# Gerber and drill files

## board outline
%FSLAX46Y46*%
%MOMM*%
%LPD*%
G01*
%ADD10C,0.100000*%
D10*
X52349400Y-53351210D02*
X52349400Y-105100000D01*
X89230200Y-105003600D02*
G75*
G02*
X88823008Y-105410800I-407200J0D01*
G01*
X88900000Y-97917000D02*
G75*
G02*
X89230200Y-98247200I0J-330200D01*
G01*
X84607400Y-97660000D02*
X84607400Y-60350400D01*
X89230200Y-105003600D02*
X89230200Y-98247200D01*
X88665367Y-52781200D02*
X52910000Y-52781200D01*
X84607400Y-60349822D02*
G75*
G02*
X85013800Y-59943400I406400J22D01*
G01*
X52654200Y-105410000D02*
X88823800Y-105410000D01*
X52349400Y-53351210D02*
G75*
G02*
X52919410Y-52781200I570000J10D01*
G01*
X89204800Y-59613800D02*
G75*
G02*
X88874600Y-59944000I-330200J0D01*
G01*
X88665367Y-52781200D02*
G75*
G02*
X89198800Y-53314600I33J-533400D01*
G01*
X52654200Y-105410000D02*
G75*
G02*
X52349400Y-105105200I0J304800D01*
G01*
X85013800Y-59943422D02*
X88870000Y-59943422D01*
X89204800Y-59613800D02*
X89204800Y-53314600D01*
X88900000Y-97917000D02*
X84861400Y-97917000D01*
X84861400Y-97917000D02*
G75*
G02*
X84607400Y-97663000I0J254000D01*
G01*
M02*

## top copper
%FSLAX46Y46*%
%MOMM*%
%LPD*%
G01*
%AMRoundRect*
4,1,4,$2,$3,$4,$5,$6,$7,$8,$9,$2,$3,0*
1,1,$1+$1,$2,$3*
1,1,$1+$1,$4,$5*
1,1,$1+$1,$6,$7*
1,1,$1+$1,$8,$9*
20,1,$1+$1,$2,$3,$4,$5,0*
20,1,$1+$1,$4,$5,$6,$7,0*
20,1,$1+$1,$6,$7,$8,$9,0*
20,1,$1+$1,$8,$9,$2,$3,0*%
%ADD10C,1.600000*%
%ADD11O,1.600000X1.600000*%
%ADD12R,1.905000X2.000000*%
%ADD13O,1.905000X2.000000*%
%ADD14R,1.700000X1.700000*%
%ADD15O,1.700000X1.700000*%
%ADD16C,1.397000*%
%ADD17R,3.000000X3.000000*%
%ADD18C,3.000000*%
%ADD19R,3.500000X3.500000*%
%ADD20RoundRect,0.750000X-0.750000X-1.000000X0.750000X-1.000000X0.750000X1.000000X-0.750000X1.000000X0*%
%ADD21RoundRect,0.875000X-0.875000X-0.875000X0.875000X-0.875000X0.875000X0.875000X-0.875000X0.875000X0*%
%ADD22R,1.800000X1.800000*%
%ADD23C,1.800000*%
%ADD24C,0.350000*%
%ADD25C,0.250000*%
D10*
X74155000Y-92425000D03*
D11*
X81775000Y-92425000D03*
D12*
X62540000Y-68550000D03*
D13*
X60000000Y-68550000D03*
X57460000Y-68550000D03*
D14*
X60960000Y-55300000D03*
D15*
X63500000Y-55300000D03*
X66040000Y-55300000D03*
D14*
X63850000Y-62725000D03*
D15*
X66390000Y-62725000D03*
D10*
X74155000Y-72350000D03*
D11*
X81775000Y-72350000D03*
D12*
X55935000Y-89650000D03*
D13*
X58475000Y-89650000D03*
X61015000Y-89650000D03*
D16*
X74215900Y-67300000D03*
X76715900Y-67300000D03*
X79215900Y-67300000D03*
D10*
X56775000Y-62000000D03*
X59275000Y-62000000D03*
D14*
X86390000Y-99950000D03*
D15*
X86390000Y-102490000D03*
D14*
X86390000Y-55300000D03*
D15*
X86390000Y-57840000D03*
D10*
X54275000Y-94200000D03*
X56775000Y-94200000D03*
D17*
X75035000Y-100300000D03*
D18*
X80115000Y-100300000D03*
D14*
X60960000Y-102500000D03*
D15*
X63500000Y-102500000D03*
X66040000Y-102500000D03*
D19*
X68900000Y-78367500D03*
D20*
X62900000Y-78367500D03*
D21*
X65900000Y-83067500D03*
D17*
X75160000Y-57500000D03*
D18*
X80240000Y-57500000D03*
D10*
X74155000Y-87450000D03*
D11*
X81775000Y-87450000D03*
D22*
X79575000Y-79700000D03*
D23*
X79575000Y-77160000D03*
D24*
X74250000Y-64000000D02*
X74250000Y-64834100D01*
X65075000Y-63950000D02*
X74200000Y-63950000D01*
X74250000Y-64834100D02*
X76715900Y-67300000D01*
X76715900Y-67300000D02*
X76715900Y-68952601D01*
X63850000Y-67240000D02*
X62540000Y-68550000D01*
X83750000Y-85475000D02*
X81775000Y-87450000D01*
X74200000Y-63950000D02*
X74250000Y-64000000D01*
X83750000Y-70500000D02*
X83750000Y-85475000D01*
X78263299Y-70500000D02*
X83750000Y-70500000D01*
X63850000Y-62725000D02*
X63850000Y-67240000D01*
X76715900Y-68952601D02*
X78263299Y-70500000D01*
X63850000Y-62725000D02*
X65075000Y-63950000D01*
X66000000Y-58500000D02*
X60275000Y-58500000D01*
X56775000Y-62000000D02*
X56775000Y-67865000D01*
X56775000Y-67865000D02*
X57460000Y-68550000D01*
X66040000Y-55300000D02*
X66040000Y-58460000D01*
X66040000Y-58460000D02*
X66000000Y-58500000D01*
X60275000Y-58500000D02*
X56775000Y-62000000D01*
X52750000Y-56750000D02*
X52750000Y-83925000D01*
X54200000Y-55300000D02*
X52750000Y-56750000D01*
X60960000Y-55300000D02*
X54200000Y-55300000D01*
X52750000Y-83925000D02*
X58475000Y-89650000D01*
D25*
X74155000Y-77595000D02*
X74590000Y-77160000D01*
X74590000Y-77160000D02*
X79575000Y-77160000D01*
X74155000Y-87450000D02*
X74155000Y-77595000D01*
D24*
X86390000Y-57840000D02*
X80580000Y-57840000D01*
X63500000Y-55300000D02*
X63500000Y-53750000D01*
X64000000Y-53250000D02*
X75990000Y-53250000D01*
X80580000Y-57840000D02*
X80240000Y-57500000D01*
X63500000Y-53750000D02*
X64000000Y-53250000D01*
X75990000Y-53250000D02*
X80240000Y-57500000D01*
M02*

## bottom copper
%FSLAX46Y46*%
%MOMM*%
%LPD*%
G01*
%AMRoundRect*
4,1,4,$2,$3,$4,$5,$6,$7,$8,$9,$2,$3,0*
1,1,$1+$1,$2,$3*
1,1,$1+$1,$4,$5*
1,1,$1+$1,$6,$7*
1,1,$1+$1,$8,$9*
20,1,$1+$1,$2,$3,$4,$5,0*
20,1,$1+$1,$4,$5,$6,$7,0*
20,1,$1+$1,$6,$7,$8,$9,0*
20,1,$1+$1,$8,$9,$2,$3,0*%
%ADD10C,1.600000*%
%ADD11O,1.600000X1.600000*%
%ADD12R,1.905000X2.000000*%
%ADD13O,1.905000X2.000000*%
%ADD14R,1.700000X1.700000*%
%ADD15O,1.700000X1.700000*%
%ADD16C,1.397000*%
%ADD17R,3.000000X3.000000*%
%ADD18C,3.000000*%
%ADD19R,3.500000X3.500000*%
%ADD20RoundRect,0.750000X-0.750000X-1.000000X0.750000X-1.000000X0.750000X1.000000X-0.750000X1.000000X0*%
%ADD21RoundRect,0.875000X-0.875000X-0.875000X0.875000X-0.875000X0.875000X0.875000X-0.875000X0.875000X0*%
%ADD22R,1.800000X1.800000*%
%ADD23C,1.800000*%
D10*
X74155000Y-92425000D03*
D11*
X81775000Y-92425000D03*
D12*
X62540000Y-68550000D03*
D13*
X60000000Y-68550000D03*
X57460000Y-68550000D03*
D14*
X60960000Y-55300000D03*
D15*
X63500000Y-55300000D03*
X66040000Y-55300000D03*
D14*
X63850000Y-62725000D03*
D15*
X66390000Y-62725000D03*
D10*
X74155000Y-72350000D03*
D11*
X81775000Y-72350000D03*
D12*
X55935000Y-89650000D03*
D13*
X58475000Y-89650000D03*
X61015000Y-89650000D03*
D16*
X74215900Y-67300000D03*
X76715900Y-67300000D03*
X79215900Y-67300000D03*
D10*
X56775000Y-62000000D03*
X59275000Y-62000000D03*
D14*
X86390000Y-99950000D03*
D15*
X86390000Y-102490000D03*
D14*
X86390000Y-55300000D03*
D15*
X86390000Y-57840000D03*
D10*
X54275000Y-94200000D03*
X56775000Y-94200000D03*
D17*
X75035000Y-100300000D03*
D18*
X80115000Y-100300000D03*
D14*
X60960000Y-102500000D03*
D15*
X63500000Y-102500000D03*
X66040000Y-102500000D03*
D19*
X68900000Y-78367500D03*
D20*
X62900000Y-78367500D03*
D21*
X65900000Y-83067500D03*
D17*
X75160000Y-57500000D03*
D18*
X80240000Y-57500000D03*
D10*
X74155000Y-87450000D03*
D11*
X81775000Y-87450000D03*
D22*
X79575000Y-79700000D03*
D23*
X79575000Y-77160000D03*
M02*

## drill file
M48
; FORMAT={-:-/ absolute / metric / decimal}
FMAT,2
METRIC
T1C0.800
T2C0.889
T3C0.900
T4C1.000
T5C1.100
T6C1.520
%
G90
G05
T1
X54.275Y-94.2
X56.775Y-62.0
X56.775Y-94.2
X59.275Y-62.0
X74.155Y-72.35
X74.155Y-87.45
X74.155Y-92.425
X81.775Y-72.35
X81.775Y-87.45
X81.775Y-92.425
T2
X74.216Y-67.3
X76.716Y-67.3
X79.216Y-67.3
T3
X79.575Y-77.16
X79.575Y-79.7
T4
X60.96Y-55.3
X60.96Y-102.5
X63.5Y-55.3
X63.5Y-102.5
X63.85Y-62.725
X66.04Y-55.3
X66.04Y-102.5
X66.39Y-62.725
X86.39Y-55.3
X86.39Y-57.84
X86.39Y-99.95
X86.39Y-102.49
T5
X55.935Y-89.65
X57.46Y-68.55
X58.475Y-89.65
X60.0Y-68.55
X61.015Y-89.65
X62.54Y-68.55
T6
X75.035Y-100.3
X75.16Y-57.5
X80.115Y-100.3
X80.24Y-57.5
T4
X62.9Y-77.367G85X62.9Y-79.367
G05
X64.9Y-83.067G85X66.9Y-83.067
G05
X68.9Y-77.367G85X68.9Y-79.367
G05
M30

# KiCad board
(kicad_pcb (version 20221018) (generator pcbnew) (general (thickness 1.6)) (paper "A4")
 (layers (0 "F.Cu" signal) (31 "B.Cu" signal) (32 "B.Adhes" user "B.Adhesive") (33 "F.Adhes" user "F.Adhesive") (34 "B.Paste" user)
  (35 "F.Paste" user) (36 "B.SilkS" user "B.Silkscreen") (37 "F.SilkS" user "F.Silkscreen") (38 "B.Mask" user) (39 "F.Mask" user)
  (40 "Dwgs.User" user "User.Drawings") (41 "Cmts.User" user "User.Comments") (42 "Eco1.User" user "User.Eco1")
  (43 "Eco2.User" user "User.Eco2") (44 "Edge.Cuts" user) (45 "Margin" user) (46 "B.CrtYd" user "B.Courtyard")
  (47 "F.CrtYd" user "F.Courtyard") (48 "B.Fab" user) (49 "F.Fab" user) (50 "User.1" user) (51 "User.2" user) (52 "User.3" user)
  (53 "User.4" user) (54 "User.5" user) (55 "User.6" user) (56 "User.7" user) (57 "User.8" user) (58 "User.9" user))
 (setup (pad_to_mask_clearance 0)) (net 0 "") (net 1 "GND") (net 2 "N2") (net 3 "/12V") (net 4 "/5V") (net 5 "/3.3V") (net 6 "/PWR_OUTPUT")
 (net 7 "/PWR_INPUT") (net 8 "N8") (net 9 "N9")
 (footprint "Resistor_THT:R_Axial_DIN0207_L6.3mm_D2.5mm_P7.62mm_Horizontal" (layer "F.Cu") (at 74.155 92.425)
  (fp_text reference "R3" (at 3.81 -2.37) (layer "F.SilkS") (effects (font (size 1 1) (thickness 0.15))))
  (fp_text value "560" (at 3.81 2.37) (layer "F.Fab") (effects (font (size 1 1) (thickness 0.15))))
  (pad "1" thru_hole circle (at 0 0) (size 1.6 1.6) (drill 0.8) (layers "*.Cu" "*.Mask") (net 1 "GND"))
  (pad "2" thru_hole oval (at 7.62 0) (size 1.6 1.6) (drill 0.8) (layers "*.Cu" "*.Mask") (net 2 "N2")))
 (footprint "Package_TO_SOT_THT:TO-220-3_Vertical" (layer "F.Cu") (at 62.54 68.55 180)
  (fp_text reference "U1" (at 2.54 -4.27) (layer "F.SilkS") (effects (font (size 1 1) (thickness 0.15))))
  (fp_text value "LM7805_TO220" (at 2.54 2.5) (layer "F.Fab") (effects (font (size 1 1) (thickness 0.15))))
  (pad "1" thru_hole rect (at 0 0 180) (size 1.905 2) (drill 1.1) (layers "*.Cu" "*.Mask") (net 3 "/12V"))
  (pad "2" thru_hole oval (at 2.54 0 180) (size 1.905 2) (drill 1.1) (layers "*.Cu" "*.Mask") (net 1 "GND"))
  (pad "3" thru_hole oval (at 5.08 0 180) (size 1.905 2) (drill 1.1) (layers "*.Cu" "*.Mask") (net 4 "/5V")))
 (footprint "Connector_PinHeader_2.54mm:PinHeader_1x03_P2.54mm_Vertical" (layer "F.Cu") (at 60.96 55.3 90)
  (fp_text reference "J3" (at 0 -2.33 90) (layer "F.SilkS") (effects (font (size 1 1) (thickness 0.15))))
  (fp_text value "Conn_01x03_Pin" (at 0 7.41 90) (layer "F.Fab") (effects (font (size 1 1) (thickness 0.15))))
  (pad "1" thru_hole rect (at 0 0 90) (size 1.7 1.7) (drill 1) (layers "*.Cu" "*.Mask") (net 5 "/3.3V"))
  (pad "2" thru_hole oval (at 0 2.54 90) (size 1.7 1.7) (drill 1) (layers "*.Cu" "*.Mask") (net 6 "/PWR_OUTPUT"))
  (pad "3" thru_hole oval (at 0 5.08 90) (size 1.7 1.7) (drill 1) (layers "*.Cu" "*.Mask") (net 4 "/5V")))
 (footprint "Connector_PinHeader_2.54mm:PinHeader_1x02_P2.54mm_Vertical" (layer "F.Cu") (at 63.85 62.725 90)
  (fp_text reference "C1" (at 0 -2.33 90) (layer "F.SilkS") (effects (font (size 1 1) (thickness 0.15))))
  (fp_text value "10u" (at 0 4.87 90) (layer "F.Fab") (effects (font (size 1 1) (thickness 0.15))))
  (pad "1" thru_hole rect (at 0 0 90) (size 1.7 1.7) (drill 1) (layers "*.Cu" "*.Mask") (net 3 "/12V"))
  (pad "2" thru_hole oval (at 0 2.54 90) (size 1.7 1.7) (drill 1) (layers "*.Cu" "*.Mask") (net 1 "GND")))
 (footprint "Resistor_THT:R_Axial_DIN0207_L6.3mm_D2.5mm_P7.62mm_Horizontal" (layer "F.Cu") (at 74.155 72.35)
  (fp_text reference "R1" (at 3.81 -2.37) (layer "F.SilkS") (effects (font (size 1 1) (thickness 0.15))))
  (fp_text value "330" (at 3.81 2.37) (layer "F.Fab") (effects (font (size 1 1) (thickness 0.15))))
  (pad "1" thru_hole circle (at 0 0) (size 1.6 1.6) (drill 0.8) (layers "*.Cu" "*.Mask") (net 2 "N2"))
  (pad "2" thru_hole oval (at 7.62 0) (size 1.6 1.6) (drill 0.8) (layers "*.Cu" "*.Mask") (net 5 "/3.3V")))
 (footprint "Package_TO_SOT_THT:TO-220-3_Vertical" (layer "F.Cu") (at 55.935 89.65)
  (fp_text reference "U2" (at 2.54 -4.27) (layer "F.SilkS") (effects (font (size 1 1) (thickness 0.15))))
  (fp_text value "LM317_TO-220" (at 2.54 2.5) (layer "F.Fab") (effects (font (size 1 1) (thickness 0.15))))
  (pad "1" thru_hole rect (at 0 0) (size 1.905 2) (drill 1.1) (layers "*.Cu" "*.Mask") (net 2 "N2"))
  (pad "2" thru_hole oval (at 2.54 0) (size 1.905 2) (drill 1.1) (layers "*.Cu" "*.Mask") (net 5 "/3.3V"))
  (pad "3" thru_hole oval (at 5.08 0) (size 1.905 2) (drill 1.1) (layers "*.Cu" "*.Mask") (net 3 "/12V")))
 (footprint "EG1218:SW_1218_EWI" (layer "F.Cu") (at 74.2159 67.3 90)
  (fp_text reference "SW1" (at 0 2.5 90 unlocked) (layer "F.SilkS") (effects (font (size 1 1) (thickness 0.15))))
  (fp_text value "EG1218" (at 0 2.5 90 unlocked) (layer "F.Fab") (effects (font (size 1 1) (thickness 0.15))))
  (pad "1" thru_hole circle (at 0 0 90) (size 1.397 1.397) (drill 0.889) (layers "*.Cu" "*.Mask") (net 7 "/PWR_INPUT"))
  (pad "2" thru_hole circle (at 0 2.5 90) (size 1.397 1.397) (drill 0.889) (layers "*.Cu" "*.Mask") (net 3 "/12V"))
  (pad "3" thru_hole circle (at 0 5 90) (size 1.397 1.397) (drill 0.889) (layers "*.Cu" "*.Mask") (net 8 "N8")))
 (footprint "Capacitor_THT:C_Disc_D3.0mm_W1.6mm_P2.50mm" (layer "F.Cu") (at 56.775 62)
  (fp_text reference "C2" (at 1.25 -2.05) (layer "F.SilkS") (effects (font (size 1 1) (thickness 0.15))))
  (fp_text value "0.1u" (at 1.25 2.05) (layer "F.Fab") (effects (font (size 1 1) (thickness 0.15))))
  (pad "1" thru_hole circle (at 0 0) (size 1.6 1.6) (drill 0.8) (layers "*.Cu" "*.Mask") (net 4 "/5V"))
  (pad "2" thru_hole circle (at 2.5 0) (size 1.6 1.6) (drill 0.8) (layers "*.Cu" "*.Mask") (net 1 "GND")))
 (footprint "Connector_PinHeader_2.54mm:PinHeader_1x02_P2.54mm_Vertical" (layer "F.Cu") (at 86.39 99.95)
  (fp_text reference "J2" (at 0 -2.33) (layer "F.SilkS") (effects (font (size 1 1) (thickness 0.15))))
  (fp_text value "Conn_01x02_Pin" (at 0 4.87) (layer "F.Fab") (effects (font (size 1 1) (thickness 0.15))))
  (pad "1" thru_hole rect (at 0 0) (size 1.7 1.7) (drill 1) (layers "*.Cu" "*.Mask") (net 1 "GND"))
  (pad "2" thru_hole oval (at 0 2.54) (size 1.7 1.7) (drill 1) (layers "*.Cu" "*.Mask") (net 6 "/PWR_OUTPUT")))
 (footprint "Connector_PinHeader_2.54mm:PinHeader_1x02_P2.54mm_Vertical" (layer "F.Cu") (at 86.39 55.3)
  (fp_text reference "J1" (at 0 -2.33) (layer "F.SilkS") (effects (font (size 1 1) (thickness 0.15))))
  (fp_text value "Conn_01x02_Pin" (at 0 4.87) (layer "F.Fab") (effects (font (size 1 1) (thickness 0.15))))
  (pad "1" thru_hole rect (at 0 0) (size 1.7 1.7) (drill 1) (layers "*.Cu" "*.Mask") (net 1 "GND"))
  (pad "2" thru_hole oval (at 0 2.54) (size 1.7 1.7) (drill 1) (layers "*.Cu" "*.Mask") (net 6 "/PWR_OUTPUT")))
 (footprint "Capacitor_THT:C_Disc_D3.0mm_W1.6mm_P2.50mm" (layer "F.Cu") (at 54.275 94.2)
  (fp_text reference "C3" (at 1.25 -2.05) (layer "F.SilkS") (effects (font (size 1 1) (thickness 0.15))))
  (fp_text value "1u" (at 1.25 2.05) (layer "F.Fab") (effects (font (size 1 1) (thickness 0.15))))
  (pad "1" thru_hole circle (at 0 0) (size 1.6 1.6) (drill 0.8) (layers "*.Cu" "*.Mask") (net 5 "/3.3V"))
  (pad "2" thru_hole circle (at 2.5 0) (size 1.6 1.6) (drill 0.8) (layers "*.Cu" "*.Mask") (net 1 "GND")))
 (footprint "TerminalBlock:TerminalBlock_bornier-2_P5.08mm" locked (layer "F.Cu") (at 75.035 100.3)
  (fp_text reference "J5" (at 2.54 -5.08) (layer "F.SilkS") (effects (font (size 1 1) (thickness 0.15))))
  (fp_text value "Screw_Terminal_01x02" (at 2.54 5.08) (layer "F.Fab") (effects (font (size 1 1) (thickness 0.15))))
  (pad "1" thru_hole rect locked (at 0 0) (size 3 3) (drill 1.52) (layers "*.Cu" "*.Mask") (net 1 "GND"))
  (pad "2" thru_hole circle locked (at 5.08 0) (size 3 3) (drill 1.52) (layers "*.Cu" "*.Mask") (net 6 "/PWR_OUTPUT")))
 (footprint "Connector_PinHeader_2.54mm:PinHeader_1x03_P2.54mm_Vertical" (layer "F.Cu") (at 60.96 102.5 90)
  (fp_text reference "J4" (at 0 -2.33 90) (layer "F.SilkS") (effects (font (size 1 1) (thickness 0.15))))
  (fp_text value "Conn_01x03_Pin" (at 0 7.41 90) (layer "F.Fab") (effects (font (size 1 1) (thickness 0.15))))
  (pad "1" thru_hole rect (at 0 0 90) (size 1.7 1.7) (drill 1) (layers "*.Cu" "*.Mask") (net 5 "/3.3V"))
  (pad "2" thru_hole oval (at 0 2.54 90) (size 1.7 1.7) (drill 1) (layers "*.Cu" "*.Mask") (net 6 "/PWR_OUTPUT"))
  (pad "3" thru_hole oval (at 0 5.08 90) (size 1.7 1.7) (drill 1) (layers "*.Cu" "*.Mask") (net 4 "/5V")))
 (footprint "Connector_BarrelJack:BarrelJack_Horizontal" (layer "F.Cu") (at 68.9 78.3675)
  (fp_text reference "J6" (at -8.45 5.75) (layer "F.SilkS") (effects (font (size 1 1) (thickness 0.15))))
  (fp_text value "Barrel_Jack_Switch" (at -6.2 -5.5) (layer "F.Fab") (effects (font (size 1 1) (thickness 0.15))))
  (pad "1" thru_hole rect (at 0 0) (size 3.5 3.5) (drill oval 1 3) (layers "*.Cu" "*.Mask") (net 7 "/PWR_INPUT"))
  (pad "2" thru_hole roundrect (at -6 0) (size 3 3.5) (drill oval 1 3) (layers "*.Cu" "*.Mask") (roundrect_rratio 0.25) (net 1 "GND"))
  (pad "3" thru_hole roundrect (at -3 4.7) (size 3.5 3.5) (drill oval 3 1) (layers "*.Cu" "*.Mask") (roundrect_rratio 0.25) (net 1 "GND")))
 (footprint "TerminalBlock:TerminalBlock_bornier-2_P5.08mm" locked (layer "F.Cu") (at 75.16 57.5)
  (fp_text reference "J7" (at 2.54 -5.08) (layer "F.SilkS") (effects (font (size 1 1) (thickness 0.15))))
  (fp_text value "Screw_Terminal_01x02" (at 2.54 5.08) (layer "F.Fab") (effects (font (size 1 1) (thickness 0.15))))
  (pad "1" thru_hole rect locked (at 0 0) (size 3 3) (drill 1.52) (layers "*.Cu" "*.Mask") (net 1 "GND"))
  (pad "2" thru_hole circle locked (at 5.08 0) (size 3 3) (drill 1.52) (layers "*.Cu" "*.Mask") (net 6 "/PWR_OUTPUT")))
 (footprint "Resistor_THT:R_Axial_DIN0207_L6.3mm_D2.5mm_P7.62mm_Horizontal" (layer "F.Cu") (at 74.155 87.45)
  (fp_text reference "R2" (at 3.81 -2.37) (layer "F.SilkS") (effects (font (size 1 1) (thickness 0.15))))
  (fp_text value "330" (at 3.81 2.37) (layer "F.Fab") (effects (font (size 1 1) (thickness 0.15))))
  (pad "1" thru_hole circle (at 0 0) (size 1.6 1.6) (drill 0.8) (layers "*.Cu" "*.Mask") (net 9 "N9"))
  (pad "2" thru_hole oval (at 7.62 0) (size 1.6 1.6) (drill 0.8) (layers "*.Cu" "*.Mask") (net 3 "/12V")))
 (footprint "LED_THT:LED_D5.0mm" (layer "F.Cu") (at 79.575 79.7 90)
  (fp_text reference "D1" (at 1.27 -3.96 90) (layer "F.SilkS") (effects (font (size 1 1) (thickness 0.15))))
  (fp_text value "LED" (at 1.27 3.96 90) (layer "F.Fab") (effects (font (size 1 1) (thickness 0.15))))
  (pad "1" thru_hole rect (at 0 0 90) (size 1.8 1.8) (drill 0.9) (layers "*.Cu" "*.Mask") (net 1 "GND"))
  (pad "2" thru_hole circle (at 2.54 0 90) (size 1.8 1.8) (drill 0.9) (layers "*.Cu" "*.Mask") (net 9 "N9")))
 (gr_line (start 52.3494 53.35121) (end 52.3494 105.1) (stroke (width 0.1) (type default)) (layer "Edge.Cuts"))
 (gr_arc (start 89.2302 105.0036) (mid 89.110936 105.291528) (end 88.823008 105.410792) (stroke (width 0.1) (type default))
  (layer "Edge.Cuts"))
 (gr_arc (start 88.9 97.917) (mid 89.133487 98.013713) (end 89.2302 98.2472) (stroke (width 0.1) (type default)) (layer "Edge.Cuts"))
 (gr_line (start 84.6074 97.66) (end 84.6074 60.3504) (stroke (width 0.1) (type default)) (layer "Edge.Cuts"))
 (gr_line (start 89.2302 105.0036) (end 89.2302 98.2472) (stroke (width 0.1) (type default)) (layer "Edge.Cuts"))
 (gr_line (start 88.665367 52.7812) (end 52.91 52.7812) (stroke (width 0.1) (type default)) (layer "Edge.Cuts"))
 (gr_arc (start 84.6074 60.349822) (mid 84.726432 60.062454) (end 85.0138 59.943422) (stroke (width 0.1) (type default)) (layer "Edge.Cuts"))
 (gr_line (start 52.6542 105.41) (end 88.8238 105.41) (stroke (width 0.1) (type default)) (layer "Edge.Cuts"))
 (gr_arc (start 52.3494 53.35121) (mid 52.516352 52.948152) (end 52.91941 52.7812) (stroke (width 0.1) (type default)) (layer "Edge.Cuts"))
 (gr_arc (start 89.2048 59.6138) (mid 89.108087 59.847287) (end 88.8746 59.944) (stroke (width 0.1) (type default)) (layer "Edge.Cuts"))
 (gr_arc (start 88.665367 52.7812) (mid 89.042538 52.937429) (end 89.198767 53.3146) (stroke (width 0.1) (type default)) (layer "Edge.Cuts"))
 (gr_arc (start 52.6542 105.41) (mid 52.438674 105.320726) (end 52.3494 105.1052) (stroke (width 0.1) (type default)) (layer "Edge.Cuts"))
 (gr_line (start 85.0138 59.943422) (end 88.87 59.943422) (stroke (width 0.1) (type default)) (layer "Edge.Cuts"))
 (gr_line (start 89.2048 59.6138) (end 89.2048 53.3146) (stroke (width 0.1) (type default)) (layer "Edge.Cuts"))
 (gr_line (start 88.9 97.917) (end 84.8614 97.917) (stroke (width 0.1) (type default)) (layer "Edge.Cuts"))
 (gr_arc (start 84.8614 97.917) (mid 84.681795 97.842605) (end 84.6074 97.663) (stroke (width 0.1) (type default)) (layer "Edge.Cuts"))
 (segment (start 74.25 64) (end 74.25 64.8341) (width 0.35) (layer "F.Cu") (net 3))
 (segment (start 65.075 63.95) (end 74.2 63.95) (width 0.35) (layer "F.Cu") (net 3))
 (segment (start 74.25 64.8341) (end 76.7159 67.3) (width 0.35) (layer "F.Cu") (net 3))
 (segment (start 76.7159 67.3) (end 76.7159 68.952601) (width 0.35) (layer "F.Cu") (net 3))
 (segment (start 63.85 67.24) (end 62.54 68.55) (width 0.35) (layer "F.Cu") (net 3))
 (segment (start 83.75 85.475) (end 81.775 87.45) (width 0.35) (layer "F.Cu") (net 3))
 (segment (start 74.2 63.95) (end 74.25 64) (width 0.35) (layer "F.Cu") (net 3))
 (segment (start 83.75 70.5) (end 83.75 85.475) (width 0.35) (layer "F.Cu") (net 3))
 (segment (start 78.263299 70.5) (end 83.75 70.5) (width 0.35) (layer "F.Cu") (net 3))
 (segment (start 63.85 62.725) (end 63.85 67.24) (width 0.35) (layer "F.Cu") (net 3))
 (segment (start 76.7159 68.952601) (end 78.263299 70.5) (width 0.35) (layer "F.Cu") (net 3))
 (segment (start 63.85 62.725) (end 65.075 63.95) (width 0.35) (layer "F.Cu") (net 3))
 (segment (start 66 58.5) (end 60.275 58.5) (width 0.35) (layer "F.Cu") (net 4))
 (segment (start 56.775 62) (end 56.775 67.865) (width 0.35) (layer "F.Cu") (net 4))
 (segment (start 56.775 67.865) (end 57.46 68.55) (width 0.35) (layer "F.Cu") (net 4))
 (segment (start 66.04 55.3) (end 66.04 58.46) (width 0.35) (layer "F.Cu") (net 4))
 (segment (start 66.04 58.46) (end 66 58.5) (width 0.35) (layer "F.Cu") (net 4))
 (segment (start 60.275 58.5) (end 56.775 62) (width 0.35) (layer "F.Cu") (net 4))
 (segment (start 52.75 56.75) (end 52.75 83.925) (width 0.35) (layer "F.Cu") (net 5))
 (segment (start 54.2 55.3) (end 52.75 56.75) (width 0.35) (layer "F.Cu") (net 5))
 (segment (start 60.96 55.3) (end 54.2 55.3) (width 0.35) (layer "F.Cu") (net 5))
 (segment (start 52.75 83.925) (end 58.475 89.65) (width 0.35) (layer "F.Cu") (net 5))
 (segment (start 74.155 77.595) (end 74.59 77.16) (width 0.25) (layer "F.Cu") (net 9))
 (segment (start 74.59 77.16) (end 79.575 77.16) (width 0.25) (layer "F.Cu") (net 9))
 (segment (start 74.155 87.45) (end 74.155 77.595) (width 0.25) (layer "F.Cu") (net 9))
 (segment (start 86.39 57.84) (end 80.58 57.84) (width 0.35) (layer "F.Cu") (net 6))
 (segment (start 63.5 55.3) (end 63.5 53.75) (width 0.35) (layer "F.Cu") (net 6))
 (segment (start 64 53.25) (end 75.99 53.25) (width 0.35) (layer "F.Cu") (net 6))
 (segment (start 80.58 57.84) (end 80.24 57.5) (width 0.35) (layer "F.Cu") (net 6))
 (segment (start 63.5 53.75) (end 64 53.25) (width 0.35) (layer "F.Cu") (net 6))
 (segment (start 75.99 53.25) (end 80.24 57.5) (width 0.35) (layer "F.Cu") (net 6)))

